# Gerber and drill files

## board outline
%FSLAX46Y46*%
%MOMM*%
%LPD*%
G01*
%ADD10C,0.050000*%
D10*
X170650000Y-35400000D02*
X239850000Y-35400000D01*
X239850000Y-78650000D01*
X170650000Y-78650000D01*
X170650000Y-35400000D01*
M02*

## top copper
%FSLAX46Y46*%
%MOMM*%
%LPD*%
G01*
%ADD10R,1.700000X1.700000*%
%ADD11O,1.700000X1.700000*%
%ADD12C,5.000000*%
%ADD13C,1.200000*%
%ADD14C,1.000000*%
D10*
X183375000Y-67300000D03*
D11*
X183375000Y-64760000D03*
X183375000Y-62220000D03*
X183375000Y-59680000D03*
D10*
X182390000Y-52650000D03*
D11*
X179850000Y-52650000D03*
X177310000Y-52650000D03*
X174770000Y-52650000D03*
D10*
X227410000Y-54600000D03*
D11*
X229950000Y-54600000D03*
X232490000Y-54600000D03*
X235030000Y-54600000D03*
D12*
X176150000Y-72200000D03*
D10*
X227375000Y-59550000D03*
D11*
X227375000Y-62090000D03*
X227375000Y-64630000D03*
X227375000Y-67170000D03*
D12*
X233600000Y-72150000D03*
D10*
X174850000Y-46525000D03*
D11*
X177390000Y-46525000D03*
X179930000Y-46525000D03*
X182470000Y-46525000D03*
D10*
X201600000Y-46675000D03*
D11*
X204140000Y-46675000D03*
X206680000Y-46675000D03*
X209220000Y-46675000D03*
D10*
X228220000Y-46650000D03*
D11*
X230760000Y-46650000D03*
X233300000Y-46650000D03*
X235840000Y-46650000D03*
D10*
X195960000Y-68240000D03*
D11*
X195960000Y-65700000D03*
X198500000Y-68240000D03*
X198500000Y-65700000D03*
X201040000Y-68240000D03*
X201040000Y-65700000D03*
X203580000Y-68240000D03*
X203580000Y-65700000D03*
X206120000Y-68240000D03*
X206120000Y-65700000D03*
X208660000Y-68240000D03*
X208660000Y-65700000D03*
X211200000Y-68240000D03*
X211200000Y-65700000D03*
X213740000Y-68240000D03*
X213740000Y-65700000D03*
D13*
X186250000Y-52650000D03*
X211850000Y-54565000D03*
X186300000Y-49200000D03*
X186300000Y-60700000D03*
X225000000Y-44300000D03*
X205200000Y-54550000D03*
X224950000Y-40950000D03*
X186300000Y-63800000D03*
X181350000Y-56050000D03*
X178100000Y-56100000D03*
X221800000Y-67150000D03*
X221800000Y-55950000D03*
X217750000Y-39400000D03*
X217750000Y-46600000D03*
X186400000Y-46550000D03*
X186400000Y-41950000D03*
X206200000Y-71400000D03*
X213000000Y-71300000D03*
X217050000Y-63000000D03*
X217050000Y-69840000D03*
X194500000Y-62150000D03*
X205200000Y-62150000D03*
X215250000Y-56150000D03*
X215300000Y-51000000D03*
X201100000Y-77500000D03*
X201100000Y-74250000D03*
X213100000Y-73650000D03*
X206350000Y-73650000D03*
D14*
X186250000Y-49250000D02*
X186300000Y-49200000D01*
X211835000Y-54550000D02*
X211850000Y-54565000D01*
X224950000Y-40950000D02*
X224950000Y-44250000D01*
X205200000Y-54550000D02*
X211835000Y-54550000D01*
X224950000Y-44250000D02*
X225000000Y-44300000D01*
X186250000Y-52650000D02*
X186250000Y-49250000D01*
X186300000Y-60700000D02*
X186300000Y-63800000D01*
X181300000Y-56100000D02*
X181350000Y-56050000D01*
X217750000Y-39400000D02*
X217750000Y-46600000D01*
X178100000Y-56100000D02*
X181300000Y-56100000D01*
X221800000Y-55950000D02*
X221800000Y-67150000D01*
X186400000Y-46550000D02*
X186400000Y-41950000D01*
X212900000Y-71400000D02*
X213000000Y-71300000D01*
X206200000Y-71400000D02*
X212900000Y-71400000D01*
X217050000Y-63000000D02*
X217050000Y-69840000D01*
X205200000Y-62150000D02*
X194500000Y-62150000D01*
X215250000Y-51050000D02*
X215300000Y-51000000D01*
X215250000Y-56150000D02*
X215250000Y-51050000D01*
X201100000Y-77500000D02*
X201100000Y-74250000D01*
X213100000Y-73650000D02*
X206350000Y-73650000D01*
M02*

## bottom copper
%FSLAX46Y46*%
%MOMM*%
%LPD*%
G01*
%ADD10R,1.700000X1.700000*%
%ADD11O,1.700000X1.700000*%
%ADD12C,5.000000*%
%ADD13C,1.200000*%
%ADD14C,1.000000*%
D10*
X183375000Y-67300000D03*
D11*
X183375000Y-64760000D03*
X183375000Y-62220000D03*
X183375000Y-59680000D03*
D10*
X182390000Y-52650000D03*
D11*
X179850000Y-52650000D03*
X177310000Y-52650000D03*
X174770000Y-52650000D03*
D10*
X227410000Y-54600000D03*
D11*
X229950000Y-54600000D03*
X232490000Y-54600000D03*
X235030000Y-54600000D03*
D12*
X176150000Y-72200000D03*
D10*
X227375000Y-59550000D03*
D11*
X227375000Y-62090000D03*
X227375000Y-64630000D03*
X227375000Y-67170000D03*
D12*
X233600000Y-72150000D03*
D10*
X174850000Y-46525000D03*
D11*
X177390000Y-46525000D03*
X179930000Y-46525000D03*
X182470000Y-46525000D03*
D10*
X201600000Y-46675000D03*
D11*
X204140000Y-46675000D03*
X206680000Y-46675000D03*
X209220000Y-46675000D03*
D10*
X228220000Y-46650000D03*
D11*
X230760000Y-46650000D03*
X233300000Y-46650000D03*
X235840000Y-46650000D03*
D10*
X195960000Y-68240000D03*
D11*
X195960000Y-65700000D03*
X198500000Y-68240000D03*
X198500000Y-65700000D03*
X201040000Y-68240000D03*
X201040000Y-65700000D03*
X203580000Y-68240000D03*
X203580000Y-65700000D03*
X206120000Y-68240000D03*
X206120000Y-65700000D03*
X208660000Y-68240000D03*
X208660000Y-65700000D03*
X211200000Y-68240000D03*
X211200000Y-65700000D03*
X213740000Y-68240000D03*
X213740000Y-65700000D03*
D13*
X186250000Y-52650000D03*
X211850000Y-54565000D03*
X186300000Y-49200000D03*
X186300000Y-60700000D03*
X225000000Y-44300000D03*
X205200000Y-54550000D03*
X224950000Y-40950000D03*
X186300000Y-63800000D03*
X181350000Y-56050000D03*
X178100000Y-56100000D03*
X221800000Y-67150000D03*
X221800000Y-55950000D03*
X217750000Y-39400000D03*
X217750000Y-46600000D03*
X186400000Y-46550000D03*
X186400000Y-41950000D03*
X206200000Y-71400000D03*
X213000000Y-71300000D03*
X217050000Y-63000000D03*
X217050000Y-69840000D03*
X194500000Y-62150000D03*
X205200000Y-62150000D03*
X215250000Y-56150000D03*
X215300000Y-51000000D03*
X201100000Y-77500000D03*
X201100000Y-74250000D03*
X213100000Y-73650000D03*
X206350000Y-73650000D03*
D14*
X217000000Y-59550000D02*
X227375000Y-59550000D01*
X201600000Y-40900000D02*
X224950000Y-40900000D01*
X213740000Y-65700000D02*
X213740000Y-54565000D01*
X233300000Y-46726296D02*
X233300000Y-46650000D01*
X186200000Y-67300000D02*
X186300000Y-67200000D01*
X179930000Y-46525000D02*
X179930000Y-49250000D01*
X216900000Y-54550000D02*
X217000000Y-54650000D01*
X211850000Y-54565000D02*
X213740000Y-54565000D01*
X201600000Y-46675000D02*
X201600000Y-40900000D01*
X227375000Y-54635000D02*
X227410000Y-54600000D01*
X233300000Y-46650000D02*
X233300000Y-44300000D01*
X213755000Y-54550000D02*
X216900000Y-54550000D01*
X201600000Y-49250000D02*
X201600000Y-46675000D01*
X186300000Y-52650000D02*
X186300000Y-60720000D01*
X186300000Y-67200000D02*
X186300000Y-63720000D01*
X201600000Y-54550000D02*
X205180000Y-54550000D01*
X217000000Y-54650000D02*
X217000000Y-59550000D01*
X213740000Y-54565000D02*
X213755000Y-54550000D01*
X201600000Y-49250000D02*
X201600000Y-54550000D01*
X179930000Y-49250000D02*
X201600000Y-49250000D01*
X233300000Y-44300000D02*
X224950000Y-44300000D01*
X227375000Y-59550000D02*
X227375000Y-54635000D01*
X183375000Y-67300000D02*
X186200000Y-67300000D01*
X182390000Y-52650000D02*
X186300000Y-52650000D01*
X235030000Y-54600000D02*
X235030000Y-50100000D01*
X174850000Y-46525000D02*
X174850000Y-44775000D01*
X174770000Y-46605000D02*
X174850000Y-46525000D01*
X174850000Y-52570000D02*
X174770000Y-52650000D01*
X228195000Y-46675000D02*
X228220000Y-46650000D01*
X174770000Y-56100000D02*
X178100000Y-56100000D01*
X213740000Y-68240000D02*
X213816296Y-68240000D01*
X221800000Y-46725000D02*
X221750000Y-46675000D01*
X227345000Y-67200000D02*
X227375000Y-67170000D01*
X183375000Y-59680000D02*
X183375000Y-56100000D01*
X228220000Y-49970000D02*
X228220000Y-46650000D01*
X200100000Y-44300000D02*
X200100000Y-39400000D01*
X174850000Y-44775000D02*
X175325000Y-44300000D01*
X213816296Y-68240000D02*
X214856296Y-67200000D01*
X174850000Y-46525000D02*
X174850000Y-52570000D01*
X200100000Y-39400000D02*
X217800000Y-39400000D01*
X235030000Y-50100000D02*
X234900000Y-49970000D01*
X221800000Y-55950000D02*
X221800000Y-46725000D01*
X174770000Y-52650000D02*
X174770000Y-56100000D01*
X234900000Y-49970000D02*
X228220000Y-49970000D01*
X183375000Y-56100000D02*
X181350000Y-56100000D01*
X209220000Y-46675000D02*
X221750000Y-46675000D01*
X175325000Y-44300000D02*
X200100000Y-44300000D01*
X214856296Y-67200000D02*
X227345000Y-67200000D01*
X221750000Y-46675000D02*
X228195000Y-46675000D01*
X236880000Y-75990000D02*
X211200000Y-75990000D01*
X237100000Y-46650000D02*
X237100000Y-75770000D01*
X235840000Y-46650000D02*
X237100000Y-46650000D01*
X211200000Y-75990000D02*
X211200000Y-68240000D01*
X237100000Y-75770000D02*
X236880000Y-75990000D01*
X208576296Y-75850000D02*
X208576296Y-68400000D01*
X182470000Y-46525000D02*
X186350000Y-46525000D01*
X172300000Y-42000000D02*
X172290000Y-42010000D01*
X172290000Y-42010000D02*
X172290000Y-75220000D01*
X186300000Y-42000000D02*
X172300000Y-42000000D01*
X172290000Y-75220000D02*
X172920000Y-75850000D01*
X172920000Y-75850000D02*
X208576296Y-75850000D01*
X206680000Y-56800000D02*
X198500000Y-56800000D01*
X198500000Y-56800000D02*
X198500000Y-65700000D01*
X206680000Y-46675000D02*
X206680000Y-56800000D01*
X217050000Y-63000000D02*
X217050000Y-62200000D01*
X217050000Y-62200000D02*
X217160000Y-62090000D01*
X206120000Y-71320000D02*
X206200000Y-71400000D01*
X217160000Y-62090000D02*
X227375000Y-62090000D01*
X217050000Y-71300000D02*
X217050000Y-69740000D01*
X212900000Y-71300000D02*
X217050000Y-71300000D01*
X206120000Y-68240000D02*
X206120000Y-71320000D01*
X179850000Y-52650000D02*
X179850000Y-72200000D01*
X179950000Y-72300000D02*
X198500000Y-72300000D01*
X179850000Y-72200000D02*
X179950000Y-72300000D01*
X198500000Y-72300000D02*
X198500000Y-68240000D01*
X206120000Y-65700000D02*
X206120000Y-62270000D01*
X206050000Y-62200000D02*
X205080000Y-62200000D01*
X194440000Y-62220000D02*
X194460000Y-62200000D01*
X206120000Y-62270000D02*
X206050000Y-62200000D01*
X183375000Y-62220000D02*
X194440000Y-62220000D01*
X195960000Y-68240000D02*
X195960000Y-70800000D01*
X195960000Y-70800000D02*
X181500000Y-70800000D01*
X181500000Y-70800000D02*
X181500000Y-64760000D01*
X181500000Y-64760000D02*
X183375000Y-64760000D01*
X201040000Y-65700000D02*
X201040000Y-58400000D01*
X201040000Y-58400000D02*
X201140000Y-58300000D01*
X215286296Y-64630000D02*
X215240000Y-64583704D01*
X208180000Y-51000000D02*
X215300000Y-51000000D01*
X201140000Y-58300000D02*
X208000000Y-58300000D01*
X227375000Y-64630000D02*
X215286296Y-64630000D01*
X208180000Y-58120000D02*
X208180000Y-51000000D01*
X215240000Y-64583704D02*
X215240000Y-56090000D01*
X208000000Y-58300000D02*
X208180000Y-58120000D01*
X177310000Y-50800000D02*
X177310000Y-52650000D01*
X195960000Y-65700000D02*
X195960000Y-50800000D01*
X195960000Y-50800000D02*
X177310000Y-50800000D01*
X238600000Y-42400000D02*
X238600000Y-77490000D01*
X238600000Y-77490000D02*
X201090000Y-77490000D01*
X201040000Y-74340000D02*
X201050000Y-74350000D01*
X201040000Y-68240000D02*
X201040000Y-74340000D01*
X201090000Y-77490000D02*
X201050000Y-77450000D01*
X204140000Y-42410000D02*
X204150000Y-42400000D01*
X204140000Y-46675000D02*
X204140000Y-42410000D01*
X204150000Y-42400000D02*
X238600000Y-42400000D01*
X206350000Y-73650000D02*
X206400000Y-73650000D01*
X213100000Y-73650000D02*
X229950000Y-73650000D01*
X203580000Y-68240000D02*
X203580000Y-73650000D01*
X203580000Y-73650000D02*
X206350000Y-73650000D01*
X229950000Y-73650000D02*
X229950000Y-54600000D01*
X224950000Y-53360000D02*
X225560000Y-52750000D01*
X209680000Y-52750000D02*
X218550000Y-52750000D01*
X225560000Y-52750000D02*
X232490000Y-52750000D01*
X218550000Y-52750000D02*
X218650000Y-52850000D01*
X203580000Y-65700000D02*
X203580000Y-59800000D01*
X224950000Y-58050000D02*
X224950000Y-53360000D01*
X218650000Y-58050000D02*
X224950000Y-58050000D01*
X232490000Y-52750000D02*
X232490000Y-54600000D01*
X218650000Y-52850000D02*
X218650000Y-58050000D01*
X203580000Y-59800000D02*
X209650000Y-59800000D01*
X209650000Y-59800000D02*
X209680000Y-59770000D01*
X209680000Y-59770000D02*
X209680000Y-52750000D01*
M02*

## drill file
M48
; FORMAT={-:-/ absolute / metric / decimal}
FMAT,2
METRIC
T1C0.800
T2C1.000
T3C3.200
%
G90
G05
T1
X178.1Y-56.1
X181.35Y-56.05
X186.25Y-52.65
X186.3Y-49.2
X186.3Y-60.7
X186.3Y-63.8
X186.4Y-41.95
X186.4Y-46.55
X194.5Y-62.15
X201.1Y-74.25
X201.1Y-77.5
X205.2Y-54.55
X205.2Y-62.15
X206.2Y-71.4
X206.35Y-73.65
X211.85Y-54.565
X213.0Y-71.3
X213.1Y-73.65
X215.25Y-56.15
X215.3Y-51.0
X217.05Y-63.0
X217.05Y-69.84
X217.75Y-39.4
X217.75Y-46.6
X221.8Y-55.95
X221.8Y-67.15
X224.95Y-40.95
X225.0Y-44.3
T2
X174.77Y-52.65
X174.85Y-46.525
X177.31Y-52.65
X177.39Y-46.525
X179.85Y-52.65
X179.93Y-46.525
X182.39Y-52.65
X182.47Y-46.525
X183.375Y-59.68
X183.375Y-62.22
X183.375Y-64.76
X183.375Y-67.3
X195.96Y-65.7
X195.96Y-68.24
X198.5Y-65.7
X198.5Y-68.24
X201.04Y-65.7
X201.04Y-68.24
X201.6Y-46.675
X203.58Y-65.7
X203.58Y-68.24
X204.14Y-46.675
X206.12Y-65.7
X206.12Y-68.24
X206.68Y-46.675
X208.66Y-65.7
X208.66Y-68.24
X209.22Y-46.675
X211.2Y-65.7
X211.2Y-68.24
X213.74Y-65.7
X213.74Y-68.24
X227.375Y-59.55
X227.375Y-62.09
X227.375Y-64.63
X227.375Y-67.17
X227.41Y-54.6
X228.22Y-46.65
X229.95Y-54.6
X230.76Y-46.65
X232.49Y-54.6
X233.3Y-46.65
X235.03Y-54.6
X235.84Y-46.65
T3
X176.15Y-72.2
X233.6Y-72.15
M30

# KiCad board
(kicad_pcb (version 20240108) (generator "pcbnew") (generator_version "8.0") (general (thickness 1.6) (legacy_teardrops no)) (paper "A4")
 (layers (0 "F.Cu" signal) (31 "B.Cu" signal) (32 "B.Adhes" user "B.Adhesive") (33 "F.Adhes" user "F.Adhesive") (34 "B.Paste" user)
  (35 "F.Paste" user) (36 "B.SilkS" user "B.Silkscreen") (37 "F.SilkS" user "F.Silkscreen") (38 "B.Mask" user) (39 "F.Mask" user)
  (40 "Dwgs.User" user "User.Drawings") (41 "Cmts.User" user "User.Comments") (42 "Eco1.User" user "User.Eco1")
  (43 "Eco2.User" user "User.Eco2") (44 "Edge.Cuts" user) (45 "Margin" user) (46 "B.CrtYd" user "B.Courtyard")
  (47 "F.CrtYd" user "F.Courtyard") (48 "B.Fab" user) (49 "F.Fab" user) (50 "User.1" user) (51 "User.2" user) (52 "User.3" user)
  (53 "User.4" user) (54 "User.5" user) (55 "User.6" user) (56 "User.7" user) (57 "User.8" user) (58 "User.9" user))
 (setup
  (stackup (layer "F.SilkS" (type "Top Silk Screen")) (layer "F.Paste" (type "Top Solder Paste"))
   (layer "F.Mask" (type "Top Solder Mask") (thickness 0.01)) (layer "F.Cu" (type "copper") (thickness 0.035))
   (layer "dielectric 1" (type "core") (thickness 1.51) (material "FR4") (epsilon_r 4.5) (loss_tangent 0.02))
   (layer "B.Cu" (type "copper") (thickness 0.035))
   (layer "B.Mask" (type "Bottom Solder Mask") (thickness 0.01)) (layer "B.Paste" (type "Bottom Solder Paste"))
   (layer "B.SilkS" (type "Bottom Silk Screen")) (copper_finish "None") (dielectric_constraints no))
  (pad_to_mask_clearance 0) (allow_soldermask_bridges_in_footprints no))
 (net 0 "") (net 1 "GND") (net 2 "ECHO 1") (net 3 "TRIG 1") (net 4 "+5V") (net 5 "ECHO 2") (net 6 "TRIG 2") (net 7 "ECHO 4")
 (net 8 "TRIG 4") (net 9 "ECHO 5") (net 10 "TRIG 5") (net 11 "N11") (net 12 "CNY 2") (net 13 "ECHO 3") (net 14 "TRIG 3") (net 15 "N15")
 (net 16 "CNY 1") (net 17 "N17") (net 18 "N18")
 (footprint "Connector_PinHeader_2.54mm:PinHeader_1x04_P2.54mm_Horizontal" (layer "F.Cu") (at 183.375 67.3 180)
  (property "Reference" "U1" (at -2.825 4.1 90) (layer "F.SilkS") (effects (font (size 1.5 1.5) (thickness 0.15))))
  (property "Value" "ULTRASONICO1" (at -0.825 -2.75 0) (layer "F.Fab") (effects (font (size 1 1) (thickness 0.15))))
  (pad "1" thru_hole rect (at 0 0 180) (size 1.7 1.7) (drill 1) (layers "*.Cu" "*.Mask") (remove_unused_layers no) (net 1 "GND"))
  (pad "2" thru_hole oval (at 0 2.54 180) (size 1.7 1.7) (drill 1) (layers "*.Cu" "*.Mask") (remove_unused_layers no) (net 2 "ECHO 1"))
  (pad "3" thru_hole oval (at 0 5.08 180) (size 1.7 1.7) (drill 1) (layers "*.Cu" "*.Mask") (remove_unused_layers no) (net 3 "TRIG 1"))
  (pad "4" thru_hole oval (at 0 7.62 180) (size 1.7 1.7) (drill 1) (layers "*.Cu" "*.Mask") (remove_unused_layers no) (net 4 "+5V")))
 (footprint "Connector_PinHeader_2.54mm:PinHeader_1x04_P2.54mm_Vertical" (layer "F.Cu") (at 182.39 52.65 -90)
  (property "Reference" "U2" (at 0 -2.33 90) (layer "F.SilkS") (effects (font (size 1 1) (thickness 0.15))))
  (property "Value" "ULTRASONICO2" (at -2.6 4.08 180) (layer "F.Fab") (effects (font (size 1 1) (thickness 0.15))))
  (pad "1" thru_hole rect (at 0 0 270) (size 1.7 1.7) (drill 1) (layers "*.Cu" "*.Mask") (remove_unused_layers no) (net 1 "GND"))
  (pad "2" thru_hole oval (at 0 2.54 270) (size 1.7 1.7) (drill 1) (layers "*.Cu" "*.Mask") (remove_unused_layers no) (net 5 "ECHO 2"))
  (pad "3" thru_hole oval (at 0 5.08 270) (size 1.7 1.7) (drill 1) (layers "*.Cu" "*.Mask") (remove_unused_layers no) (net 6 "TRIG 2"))
  (pad "4" thru_hole oval (at 0 7.62 270) (size 1.7 1.7) (drill 1) (layers "*.Cu" "*.Mask") (remove_unused_layers no) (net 4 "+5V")))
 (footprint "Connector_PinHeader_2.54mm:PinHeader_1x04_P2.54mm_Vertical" (layer "F.Cu") (at 227.41 54.6 90)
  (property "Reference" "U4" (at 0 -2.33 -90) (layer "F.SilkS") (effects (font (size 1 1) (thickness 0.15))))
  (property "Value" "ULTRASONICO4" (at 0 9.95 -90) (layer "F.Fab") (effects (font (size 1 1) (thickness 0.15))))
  (pad "1" thru_hole rect (at 0 0 90) (size 1.7 1.7) (drill 1) (layers "*.Cu" "*.Mask") (remove_unused_layers no) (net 1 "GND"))
  (pad "2" thru_hole oval (at 0 2.54 90) (size 1.7 1.7) (drill 1) (layers "*.Cu" "*.Mask") (remove_unused_layers no) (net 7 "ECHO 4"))
  (pad "3" thru_hole oval (at 0 5.08 90) (size 1.7 1.7) (drill 1) (layers "*.Cu" "*.Mask") (remove_unused_layers no) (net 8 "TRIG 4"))
  (pad "4" thru_hole oval (at 0 7.62 90) (size 1.7 1.7) (drill 1) (layers "*.Cu" "*.Mask") (remove_unused_layers no) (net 4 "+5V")))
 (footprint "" (layer "F.Cu") (at 176.15 72.2)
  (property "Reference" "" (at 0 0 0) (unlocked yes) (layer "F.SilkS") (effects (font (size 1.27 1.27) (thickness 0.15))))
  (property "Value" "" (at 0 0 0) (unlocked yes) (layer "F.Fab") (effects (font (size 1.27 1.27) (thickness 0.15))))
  (pad "1" thru_hole circle (at 0 0) (size 5 5) (drill 3.2) (layers "*.Cu" "*.Mask") (remove_unused_layers no)))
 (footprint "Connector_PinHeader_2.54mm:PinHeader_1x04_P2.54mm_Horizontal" (layer "F.Cu") (at 227.375 59.55)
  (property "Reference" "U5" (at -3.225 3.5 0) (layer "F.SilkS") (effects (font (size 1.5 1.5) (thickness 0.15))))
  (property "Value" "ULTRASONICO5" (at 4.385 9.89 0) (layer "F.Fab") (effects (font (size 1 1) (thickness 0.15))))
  (pad "1" thru_hole rect (at 0 0) (size 1.7 1.7) (drill 1) (layers "*.Cu" "*.Mask") (remove_unused_layers no) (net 1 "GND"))
  (pad "2" thru_hole oval (at 0 2.54) (size 1.7 1.7) (drill 1) (layers "*.Cu" "*.Mask") (remove_unused_layers no) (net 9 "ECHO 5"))
  (pad "3" thru_hole oval (at 0 5.08) (size 1.7 1.7) (drill 1) (layers "*.Cu" "*.Mask") (remove_unused_layers no) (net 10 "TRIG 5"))
  (pad "4" thru_hole oval (at 0 7.62) (size 1.7 1.7) (drill 1) (layers "*.Cu" "*.Mask") (remove_unused_layers no) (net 4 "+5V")))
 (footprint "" (layer "F.Cu") (at 233.6 72.15)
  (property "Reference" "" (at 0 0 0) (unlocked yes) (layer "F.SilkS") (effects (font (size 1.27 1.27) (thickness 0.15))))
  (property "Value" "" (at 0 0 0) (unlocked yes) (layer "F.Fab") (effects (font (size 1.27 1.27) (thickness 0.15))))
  (pad "1" thru_hole circle (at 0 0) (size 5 5) (drill 3.2) (layers "*.Cu" "*.Mask") (remove_unused_layers no)))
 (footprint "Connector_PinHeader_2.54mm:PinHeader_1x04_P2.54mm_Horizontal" (layer "F.Cu") (at 174.85 46.525 90)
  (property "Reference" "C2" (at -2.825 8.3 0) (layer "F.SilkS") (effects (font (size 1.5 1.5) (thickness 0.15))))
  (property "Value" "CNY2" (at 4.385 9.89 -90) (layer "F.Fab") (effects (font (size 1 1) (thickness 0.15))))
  (pad "1" thru_hole rect (at 0 0 90) (size 1.7 1.7) (drill 1) (layers "*.Cu" "*.Mask") (remove_unused_layers no) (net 4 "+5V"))
  (pad "2" thru_hole oval (at 0 2.54 90) (size 1.7 1.7) (drill 1) (layers "*.Cu" "*.Mask") (remove_unused_layers no) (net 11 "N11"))
  (pad "3" thru_hole oval (at 0 5.08 90) (size 1.7 1.7) (drill 1) (layers "*.Cu" "*.Mask") (remove_unused_layers no) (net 1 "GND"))
  (pad "4" thru_hole oval (at 0 7.62 90) (size 1.7 1.7) (drill 1) (layers "*.Cu" "*.Mask") (remove_unused_layers no) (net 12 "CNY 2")))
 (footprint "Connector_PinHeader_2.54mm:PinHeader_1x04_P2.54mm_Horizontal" (layer "F.Cu") (at 201.6 46.675 90)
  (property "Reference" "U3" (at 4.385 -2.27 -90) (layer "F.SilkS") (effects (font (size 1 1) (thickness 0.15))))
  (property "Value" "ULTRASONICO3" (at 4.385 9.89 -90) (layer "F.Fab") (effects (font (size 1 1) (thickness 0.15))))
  (pad "1" thru_hole rect (at 0 0 90) (size 1.7 1.7) (drill 1) (layers "*.Cu" "*.Mask") (remove_unused_layers no) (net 1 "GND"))
  (pad "2" thru_hole oval (at 0 2.54 90) (size 1.7 1.7) (drill 1) (layers "*.Cu" "*.Mask") (remove_unused_layers no) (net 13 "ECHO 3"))
  (pad "3" thru_hole oval (at 0 5.08 90) (size 1.7 1.7) (drill 1) (layers "*.Cu" "*.Mask") (remove_unused_layers no) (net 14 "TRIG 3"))
  (pad "4" thru_hole oval (at 0 7.62 90) (size 1.7 1.7) (drill 1) (layers "*.Cu" "*.Mask") (remove_unused_layers no) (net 4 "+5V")))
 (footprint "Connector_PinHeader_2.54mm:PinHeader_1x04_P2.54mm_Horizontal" (layer "F.Cu") (at 228.22 46.65 90)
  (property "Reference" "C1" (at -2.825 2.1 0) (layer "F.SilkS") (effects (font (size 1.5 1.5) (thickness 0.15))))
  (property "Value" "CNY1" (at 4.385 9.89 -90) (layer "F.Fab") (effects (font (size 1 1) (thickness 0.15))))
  (pad "1" thru_hole rect (at 0 0 90) (size 1.7 1.7) (drill 1) (layers "*.Cu" "*.Mask") (remove_unused_layers no) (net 4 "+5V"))
  (pad "2" thru_hole oval (at 0 2.54 90) (size 1.7 1.7) (drill 1) (layers "*.Cu" "*.Mask") (remove_unused_layers no) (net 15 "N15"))
  (pad "3" thru_hole oval (at 0 5.08 90) (size 1.7 1.7) (drill 1) (layers "*.Cu" "*.Mask") (remove_unused_layers no) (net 1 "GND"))
  (pad "4" thru_hole oval (at 0 7.62 90) (size 1.7 1.7) (drill 1) (layers "*.Cu" "*.Mask") (remove_unused_layers no) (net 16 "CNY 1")))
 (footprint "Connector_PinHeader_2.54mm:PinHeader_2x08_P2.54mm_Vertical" (layer "F.Cu") (at 195.96 68.24 90)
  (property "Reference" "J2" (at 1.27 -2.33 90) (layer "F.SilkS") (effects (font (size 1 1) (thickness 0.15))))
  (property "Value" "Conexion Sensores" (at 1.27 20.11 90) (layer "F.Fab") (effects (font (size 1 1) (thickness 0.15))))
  (pad "1" thru_hole rect (at 0 0 90) (size 1.7 1.7) (drill 1) (layers "*.Cu" "*.Mask") (remove_unused_layers no) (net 2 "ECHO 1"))
  (pad "2" thru_hole oval (at 2.54 0 90) (size 1.7 1.7) (drill 1) (layers "*.Cu" "*.Mask") (remove_unused_layers no) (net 6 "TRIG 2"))
  (pad "3" thru_hole oval (at 0 2.54 90) (size 1.7 1.7) (drill 1) (layers "*.Cu" "*.Mask") (remove_unused_layers no) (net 5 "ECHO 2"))
  (pad "4" thru_hole oval (at 2.54 2.54 90) (size 1.7 1.7) (drill 1) (layers "*.Cu" "*.Mask") (remove_unused_layers no) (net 14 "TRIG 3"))
  (pad "5" thru_hole oval (at 0 5.08 90) (size 1.7 1.7) (drill 1) (layers "*.Cu" "*.Mask") (remove_unused_layers no) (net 13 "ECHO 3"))
  (pad "6" thru_hole oval (at 2.54 5.08 90) (size 1.7 1.7) (drill 1) (layers "*.Cu" "*.Mask") (remove_unused_layers no) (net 10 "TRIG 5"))
  (pad "7" thru_hole oval (at 0 7.62 90) (size 1.7 1.7) (drill 1) (layers "*.Cu" "*.Mask") (remove_unused_layers no) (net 7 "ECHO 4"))
  (pad "8" thru_hole oval (at 2.54 7.62 90) (size 1.7 1.7) (drill 1) (layers "*.Cu" "*.Mask") (remove_unused_layers no) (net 8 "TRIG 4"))
  (pad "9" thru_hole oval (at 0 10.16 90) (size 1.7 1.7) (drill 1) (layers "*.Cu" "*.Mask") (remove_unused_layers no) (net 9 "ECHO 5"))
  (pad "10" thru_hole oval (at 2.54 10.16 90) (size 1.7 1.7) (drill 1) (layers "*.Cu" "*.Mask") (remove_unused_layers no) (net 3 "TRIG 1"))
  (pad "11" thru_hole oval (at 0 12.7 90) (size 1.7 1.7) (drill 1) (layers "*.Cu" "*.Mask") (remove_unused_layers no) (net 12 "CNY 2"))
  (pad "12" thru_hole oval (at 2.54 12.7 90) (size 1.7 1.7) (drill 1) (layers "*.Cu" "*.Mask") (remove_unused_layers no) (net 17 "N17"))
  (pad "13" thru_hole oval (at 0 15.24 90) (size 1.7 1.7) (drill 1) (layers "*.Cu" "*.Mask") (remove_unused_layers no) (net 16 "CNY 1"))
  (pad "14" thru_hole oval (at 2.54 15.24 90) (size 1.7 1.7) (drill 1) (layers "*.Cu" "*.Mask") (remove_unused_layers no) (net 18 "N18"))
  (pad "15" thru_hole oval (at 0 17.78 90) (size 1.7 1.7) (drill 1) (layers "*.Cu" "*.Mask") (remove_unused_layers no) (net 4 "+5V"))
  (pad "16" thru_hole oval (at 2.54 17.78 90) (size 1.7 1.7) (drill 1) (layers "*.Cu" "*.Mask") (remove_unused_layers no) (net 1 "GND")))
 (gr_rect (start 170.65 35.4) (end 239.85 78.65) (stroke (width 0.05) (type default)) (fill none) (layer "Edge.Cuts"))
 (segment (start 186.25 49.25) (end 186.3 49.2) (width 1) (layer "F.Cu") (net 1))
 (segment (start 211.835 54.55) (end 211.85 54.565) (width 1) (layer "F.Cu") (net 1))
 (segment (start 224.95 40.95) (end 224.95 44.25) (width 1) (layer "F.Cu") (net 1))
 (segment (start 205.2 54.55) (end 211.835 54.55) (width 1) (layer "F.Cu") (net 1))
 (segment (start 224.95 44.25) (end 225 44.3) (width 1) (layer "F.Cu") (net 1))
 (segment (start 186.25 52.65) (end 186.25 49.25) (width 1) (layer "F.Cu") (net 1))
 (segment (start 186.3 60.7) (end 186.3 63.8) (width 1) (layer "F.Cu") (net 1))
 (via (at 186.25 52.65) (size 1.2) (drill 0.8) (layers "F.Cu" "B.Cu") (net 1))
 (via (at 211.85 54.565) (size 1.2) (drill 0.8) (layers "F.Cu" "B.Cu") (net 1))
 (via (at 186.3 49.2) (size 1.2) (drill 0.8) (layers "F.Cu" "B.Cu") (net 1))
 (via (at 186.3 60.7) (size 1.2) (drill 0.8) (layers "F.Cu" "B.Cu") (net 1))
 (via (at 225 44.3) (size 1.2) (drill 0.8) (layers "F.Cu" "B.Cu") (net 1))
 (via (at 205.2 54.55) (size 1.2) (drill 0.8) (layers "F.Cu" "B.Cu") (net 1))
 (via (at 224.95 40.95) (size 1.2) (drill 0.8) (layers "F.Cu" "B.Cu") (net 1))
 (via (at 186.3 63.8) (size 1.2) (drill 0.8) (layers "F.Cu" "B.Cu") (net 1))
 (segment (start 217 59.55) (end 227.375 59.55) (width 1) (layer "B.Cu") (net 1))
 (segment (start 201.6 40.9) (end 224.95 40.9) (width 1) (layer "B.Cu") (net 1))
 (segment (start 213.74 65.7) (end 213.74 54.565) (width 1) (layer "B.Cu") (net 1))
 (segment (start 233.3 46.726296) (end 233.3 46.65) (width 1) (layer "B.Cu") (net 1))
 (segment (start 186.2 67.3) (end 186.3 67.2) (width 1) (layer "B.Cu") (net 1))
 (segment (start 179.93 46.525) (end 179.93 49.25) (width 1) (layer "B.Cu") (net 1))
 (segment (start 216.9 54.55) (end 217 54.65) (width 1) (layer "B.Cu") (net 1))
 (segment (start 211.85 54.565) (end 213.74 54.565) (width 1) (layer "B.Cu") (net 1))
 (segment (start 201.6 46.675) (end 201.6 40.9) (width 1) (layer "B.Cu") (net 1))
 (segment (start 227.375 54.635) (end 227.41 54.6) (width 1) (layer "B.Cu") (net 1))
 (segment (start 233.3 46.65) (end 233.3 44.3) (width 1) (layer "B.Cu") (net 1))
 (segment (start 213.755 54.55) (end 216.9 54.55) (width 1) (layer "B.Cu") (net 1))
 (segment (start 201.6 49.25) (end 201.6 46.675) (width 1) (layer "B.Cu") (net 1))
 (segment (start 186.3 52.65) (end 186.3 60.72) (width 1) (layer "B.Cu") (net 1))
 (segment (start 186.3 67.2) (end 186.3 63.72) (width 1) (layer "B.Cu") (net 1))
 (segment (start 201.6 54.55) (end 205.18 54.55) (width 1) (layer "B.Cu") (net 1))
 (segment (start 217 54.65) (end 217 59.55) (width 1) (layer "B.Cu") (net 1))
 (segment (start 213.74 54.565) (end 213.755 54.55) (width 1) (layer "B.Cu") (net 1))
 (segment (start 201.6 49.25) (end 201.6 54.55) (width 1) (layer "B.Cu") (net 1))
 (segment (start 179.93 49.25) (end 201.6 49.25) (width 1) (layer "B.Cu") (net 1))
 (segment (start 233.3 44.3) (end 224.95 44.3) (width 1) (layer "B.Cu") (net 1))
 (segment (start 227.375 59.55) (end 227.375 54.635) (width 1) (layer "B.Cu") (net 1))
 (segment (start 183.375 67.3) (end 186.2 67.3) (width 1) (layer "B.Cu") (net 1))
 (segment (start 182.39 52.65) (end 186.3 52.65) (width 1) (layer "B.Cu") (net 1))
 (segment (start 181.3 56.1) (end 181.35 56.05) (width 1) (layer "F.Cu") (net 4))
 (segment (start 217.75 39.4) (end 217.75 46.6) (width 1) (layer "F.Cu") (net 4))
 (segment (start 178.1 56.1) (end 181.3 56.1) (width 1) (layer "F.Cu") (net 4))
 (segment (start 221.8 55.95) (end 221.8 67.15) (width 1) (layer "F.Cu") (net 4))
 (via (at 181.35 56.05) (size 1.2) (drill 0.8) (layers "F.Cu" "B.Cu") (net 4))
 (via (at 178.1 56.1) (size 1.2) (drill 0.8) (layers "F.Cu" "B.Cu") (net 4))
 (via (at 221.8 67.15) (size 1.2) (drill 0.8) (layers "F.Cu" "B.Cu") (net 4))
 (via (at 221.8 55.95) (size 1.2) (drill 0.8) (layers "F.Cu" "B.Cu") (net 4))
 (via (at 217.75 39.4) (size 1.2) (drill 0.8) (layers "F.Cu" "B.Cu") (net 4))
 (via (at 217.75 46.6) (size 1.2) (drill 0.8) (layers "F.Cu" "B.Cu") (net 4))
 (segment (start 235.03 54.6) (end 235.03 50.1) (width 1) (layer "B.Cu") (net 4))
 (segment (start 174.85 46.525) (end 174.85 44.775) (width 1) (layer "B.Cu") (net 4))
 (segment (start 174.77 46.605) (end 174.85 46.525) (width 1) (layer "B.Cu") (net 4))
 (segment (start 174.85 52.57) (end 174.77 52.65) (width 1) (layer "B.Cu") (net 4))
 (segment (start 228.195 46.675) (end 228.22 46.65) (width 1) (layer "B.Cu") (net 4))
 (segment (start 174.77 56.1) (end 178.1 56.1) (width 1) (layer "B.Cu") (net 4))
 (segment (start 213.74 68.24) (end 213.816296 68.24) (width 1) (layer "B.Cu") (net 4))
 (segment (start 221.8 46.725) (end 221.75 46.675) (width 1) (layer "B.Cu") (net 4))
 (segment (start 227.345 67.2) (end 227.375 67.17) (width 1) (layer "B.Cu") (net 4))
 (segment (start 183.375 59.68) (end 183.375 56.1) (width 1) (layer "B.Cu") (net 4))
 (segment (start 228.22 49.97) (end 228.22 46.65) (width 1) (layer "B.Cu") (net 4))
 (segment (start 200.1 44.3) (end 200.1 39.4) (width 1) (layer "B.Cu") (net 4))
 (segment (start 174.85 44.775) (end 175.325 44.3) (width 1) (layer "B.Cu") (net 4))
 (segment (start 213.816296 68.24) (end 214.856296 67.2) (width 1) (layer "B.Cu") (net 4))
 (segment (start 174.85 46.525) (end 174.85 52.57) (width 1) (layer "B.Cu") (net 4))
 (segment (start 200.1 39.4) (end 217.8 39.4) (width 1) (layer "B.Cu") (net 4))
 (segment (start 235.03 50.1) (end 234.9 49.97) (width 1) (layer "B.Cu") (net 4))
 (segment (start 221.8 55.95) (end 221.8 46.725) (width 1) (layer "B.Cu") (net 4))
 (segment (start 174.77 52.65) (end 174.77 56.1) (width 1) (layer "B.Cu") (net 4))
 (segment (start 234.9 49.97) (end 228.22 49.97) (width 1) (layer "B.Cu") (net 4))
 (segment (start 183.375 56.1) (end 181.35 56.1) (width 1) (layer "B.Cu") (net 4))
 (segment (start 209.22 46.675) (end 221.75 46.675) (width 1) (layer "B.Cu") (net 4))
 (segment (start 175.325 44.3) (end 200.1 44.3) (width 1) (layer "B.Cu") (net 4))
 (segment (start 214.856296 67.2) (end 227.345 67.2) (width 1) (layer "B.Cu") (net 4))
 (segment (start 221.75 46.675) (end 228.195 46.675) (width 1) (layer "B.Cu") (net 4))
 (segment (start 236.88 75.99) (end 211.2 75.99) (width 1) (layer "B.Cu") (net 16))
 (segment (start 237.1 46.65) (end 237.1 75.77) (width 1) (layer "B.Cu") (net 16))
 (segment (start 235.84 46.65) (end 237.1 46.65) (width 1) (layer "B.Cu") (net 16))
 (segment (start 211.2 75.99) (end 211.2 68.24) (width 1) (layer "B.Cu") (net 16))
 (segment (start 237.1 75.77) (end 236.88 75.99) (width 1) (layer "B.Cu") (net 16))
 (segment (start 186.4 46.55) (end 186.4 41.95) (width 1) (layer "F.Cu") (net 12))
 (via (at 186.4 46.55) (size 1.2) (drill 0.8) (layers "F.Cu" "B.Cu") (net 12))
 (via (at 186.4 41.95) (size 1.2) (drill 0.8) (layers "F.Cu" "B.Cu") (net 12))
 (segment (start 208.576296 75.85) (end 208.576296 68.4) (width 1) (layer "B.Cu") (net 12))
 (segment (start 182.47 46.525) (end 186.35 46.525) (width 1) (layer "B.Cu") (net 12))
 (segment (start 172.3 42) (end 172.29 42.01) (width 1) (layer "B.Cu") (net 12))
 (segment (start 172.29 42.01) (end 172.29 75.22) (width 1) (layer "B.Cu") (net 12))
 (segment (start 186.3 42) (end 172.3 42) (width 1) (layer "B.Cu") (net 12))
 (segment (start 172.29 75.22) (end 172.92 75.85) (width 1) (layer "B.Cu") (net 12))
 (segment (start 172.92 75.85) (end 208.576296 75.85) (width 1) (layer "B.Cu") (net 12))
 (segment (start 206.68 56.8) (end 198.5 56.8) (width 1) (layer "B.Cu") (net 14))
 (segment (start 198.5 56.8) (end 198.5 65.7) (width 1) (layer "B.Cu") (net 14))
 (segment (start 206.68 46.675) (end 206.68 56.8) (width 1) (layer "B.Cu") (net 14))
 (segment (start 212.9 71.4) (end 213 71.3) (width 1) (layer "F.Cu") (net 9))
 (segment (start 206.2 71.4) (end 212.9 71.4) (width 1) (layer "F.Cu") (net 9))
 (segment (start 217.05 63) (end 217.05 69.84) (width 1) (layer "F.Cu") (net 9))
 (via (at 206.2 71.4) (size 1.2) (drill 0.8) (layers "F.Cu" "B.Cu") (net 9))
 (via (at 213 71.3) (size 1.2) (drill 0.8) (layers "F.Cu" "B.Cu") (free yes) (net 9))
 (via (at 217.05 63) (size 1.2) (drill 0.8) (layers "F.Cu" "B.Cu") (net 9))
 (via (at 217.05 69.84) (size 1.2) (drill 0.8) (layers "F.Cu" "B.Cu") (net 9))
 (segment (start 217.05 63) (end 217.05 62.2) (width 1) (layer "B.Cu") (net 9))
 (segment (start 217.05 62.2) (end 217.16 62.09) (width 1) (layer "B.Cu") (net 9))
 (segment (start 206.12 71.32) (end 206.2 71.4) (width 1) (layer "B.Cu") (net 9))
 (segment (start 217.16 62.09) (end 227.375 62.09) (width 1) (layer "B.Cu") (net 9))
 (segment (start 217.05 71.3) (end 217.05 69.74) (width 1) (layer "B.Cu") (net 9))
 (segment (start 212.9 71.3) (end 217.05 71.3) (width 1) (layer "B.Cu") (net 9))
 (segment (start 206.12 68.24) (end 206.12 71.32) (width 1) (layer "B.Cu") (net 9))
 (segment (start 179.85 52.65) (end 179.85 72.2) (width 1) (layer "B.Cu") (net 5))
 (segment (start 179.95 72.3) (end 198.5 72.3) (width 1) (layer "B.Cu") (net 5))
 (segment (start 179.85 72.2) (end 179.95 72.3) (width 1) (layer "B.Cu") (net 5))
 (segment (start 198.5 72.3) (end 198.5 68.24) (width 1) (layer "B.Cu") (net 5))
 (segment (start 205.2 62.15) (end 194.5 62.15) (width 1) (layer "F.Cu") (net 3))
 (via (at 194.5 62.15) (size 1.2) (drill 0.8) (layers "F.Cu" "B.Cu") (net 3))
 (via (at 205.2 62.15) (size 1.2) (drill 0.8) (layers "F.Cu" "B.Cu") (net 3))
 (segment (start 206.12 65.7) (end 206.12 62.27) (width 1) (layer "B.Cu") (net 3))
 (segment (start 206.05 62.2) (end 205.08 62.2) (width 1) (layer "B.Cu") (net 3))
 (segment (start 194.44 62.22) (end 194.46 62.2) (width 1) (layer "B.Cu") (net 3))
 (segment (start 206.12 62.27) (end 206.05 62.2) (width 1) (layer "B.Cu") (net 3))
 (segment (start 183.375 62.22) (end 194.44 62.22) (width 1) (layer "B.Cu") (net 3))
 (segment (start 195.96 68.24) (end 195.96 70.8) (width 1) (layer "B.Cu") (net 2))
 (segment (start 195.96 70.8) (end 181.5 70.8) (width 1) (layer "B.Cu") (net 2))
 (segment (start 181.5 70.8) (end 181.5 64.76) (width 1) (layer "B.Cu") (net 2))
 (segment (start 181.5 64.76) (end 183.375 64.76) (width 1) (layer "B.Cu") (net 2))
 (segment (start 215.25 51.05) (end 215.3 51) (width 1) (layer "F.Cu") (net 10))
 (segment (start 215.25 56.15) (end 215.25 51.05) (width 1) (layer "F.Cu") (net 10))
 (via (at 215.25 56.15) (size 1.2) (drill 0.8) (layers "F.Cu" "B.Cu") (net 10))
 (via (at 215.3 51) (size 1.2) (drill 0.8) (layers "F.Cu" "B.Cu") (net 10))
 (segment (start 201.04 65.7) (end 201.04 58.4) (width 1) (layer "B.Cu") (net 10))
 (segment (start 201.04 58.4) (end 201.14 58.3) (width 1) (layer "B.Cu") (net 10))
 (segment (start 215.286296 64.63) (end 215.24 64.583704) (width 1) (layer "B.Cu") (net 10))
 (segment (start 208.18 51) (end 215.3 51) (width 1) (layer "B.Cu") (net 10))
 (segment (start 201.14 58.3) (end 208 58.3) (width 1) (layer "B.Cu") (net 10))
 (segment (start 227.375 64.63) (end 215.286296 64.63) (width 1) (layer "B.Cu") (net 10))
 (segment (start 208.18 58.12) (end 208.18 51) (width 1) (layer "B.Cu") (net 10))
 (segment (start 215.24 64.583704) (end 215.24 56.09) (width 1) (layer "B.Cu") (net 10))
 (segment (start 208 58.3) (end 208.18 58.12) (width 1) (layer "B.Cu") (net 10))
 (segment (start 177.31 50.8) (end 177.31 52.65) (width 1) (layer "B.Cu") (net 6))
 (segment (start 195.96 65.7) (end 195.96 50.8) (width 1) (layer "B.Cu") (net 6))
 (segment (start 195.96 50.8) (end 177.31 50.8) (width 1) (layer "B.Cu") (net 6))
 (segment (start 201.1 77.5) (end 201.1 74.25) (width 1) (layer "F.Cu") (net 13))
 (via (at 201.1 77.5) (size 1.2) (drill 0.8) (layers "F.Cu" "B.Cu") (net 13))
 (via (at 201.1 74.25) (size 1.2) (drill 0.8) (layers "F.Cu" "B.Cu") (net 13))
 (segment (start 238.6 42.4) (end 238.6 77.49) (width 1) (layer "B.Cu") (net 13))
 (segment (start 238.6 77.49) (end 201.09 77.49) (width 1) (layer "B.Cu") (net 13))
 (segment (start 201.04 74.34) (end 201.05 74.35) (width 1) (layer "B.Cu") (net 13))
 (segment (start 201.04 68.24) (end 201.04 74.34) (width 1) (layer "B.Cu") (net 13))
 (segment (start 201.09 77.49) (end 201.05 77.45) (width 1) (layer "B.Cu") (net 13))
 (segment (start 204.14 42.41) (end 204.15 42.4) (width 1) (layer "B.Cu") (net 13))
 (segment (start 204.14 46.675) (end 204.14 42.41) (width 1) (layer "B.Cu") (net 13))
 (segment (start 204.15 42.4) (end 238.6 42.4) (width 1) (layer "B.Cu") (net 13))
 (segment (start 213.1 73.65) (end 206.35 73.65) (width 1) (layer "F.Cu") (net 7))
 (via (at 213.1 73.65) (size 1.2) (drill 0.8) (layers "F.Cu" "B.Cu") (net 7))
 (via (at 206.35 73.65) (size 1.2) (drill 0.8) (layers "F.Cu" "B.Cu") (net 7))
 (segment (start 206.35 73.65) (end 206.4 73.65) (width 1) (layer "B.Cu") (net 7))
 (segment (start 213.1 73.65) (end 229.95 73.65) (width 1) (layer "B.Cu") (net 7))
 (segment (start 203.58 68.24) (end 203.58 73.65) (width 1) (layer "B.Cu") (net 7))
 (segment (start 203.58 73.65) (end 206.35 73.65) (width 1) (layer "B.Cu") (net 7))
 (segment (start 229.95 73.65) (end 229.95 54.6) (width 1) (layer "B.Cu") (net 7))
 (segment (start 224.95 53.36) (end 225.56 52.75) (width 1) (layer "B.Cu") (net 8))
 (segment (start 209.68 52.75) (end 218.55 52.75) (width 1) (layer "B.Cu") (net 8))
 (segment (start 225.56 52.75) (end 232.49 52.75) (width 1) (layer "B.Cu") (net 8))
 (segment (start 218.55 52.75) (end 218.65 52.85) (width 1) (layer "B.Cu") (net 8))
 (segment (start 203.58 65.7) (end 203.58 59.8) (width 1) (layer "B.Cu") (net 8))
 (segment (start 224.95 58.05) (end 224.95 53.36) (width 1) (layer "B.Cu") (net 8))
 (segment (start 218.65 58.05) (end 224.95 58.05) (width 1) (layer "B.Cu") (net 8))
 (segment (start 232.49 52.75) (end 232.49 54.6) (width 1) (layer "B.Cu") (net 8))
 (segment (start 218.65 52.85) (end 218.65 58.05) (width 1) (layer "B.Cu") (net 8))
 (segment (start 203.58 59.8) (end 209.65 59.8) (width 1) (layer "B.Cu") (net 8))
 (segment (start 209.65 59.8) (end 209.68 59.77) (width 1) (layer "B.Cu") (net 8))
 (segment (start 209.68 59.77) (end 209.68 52.75) (width 1) (layer "B.Cu") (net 8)))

